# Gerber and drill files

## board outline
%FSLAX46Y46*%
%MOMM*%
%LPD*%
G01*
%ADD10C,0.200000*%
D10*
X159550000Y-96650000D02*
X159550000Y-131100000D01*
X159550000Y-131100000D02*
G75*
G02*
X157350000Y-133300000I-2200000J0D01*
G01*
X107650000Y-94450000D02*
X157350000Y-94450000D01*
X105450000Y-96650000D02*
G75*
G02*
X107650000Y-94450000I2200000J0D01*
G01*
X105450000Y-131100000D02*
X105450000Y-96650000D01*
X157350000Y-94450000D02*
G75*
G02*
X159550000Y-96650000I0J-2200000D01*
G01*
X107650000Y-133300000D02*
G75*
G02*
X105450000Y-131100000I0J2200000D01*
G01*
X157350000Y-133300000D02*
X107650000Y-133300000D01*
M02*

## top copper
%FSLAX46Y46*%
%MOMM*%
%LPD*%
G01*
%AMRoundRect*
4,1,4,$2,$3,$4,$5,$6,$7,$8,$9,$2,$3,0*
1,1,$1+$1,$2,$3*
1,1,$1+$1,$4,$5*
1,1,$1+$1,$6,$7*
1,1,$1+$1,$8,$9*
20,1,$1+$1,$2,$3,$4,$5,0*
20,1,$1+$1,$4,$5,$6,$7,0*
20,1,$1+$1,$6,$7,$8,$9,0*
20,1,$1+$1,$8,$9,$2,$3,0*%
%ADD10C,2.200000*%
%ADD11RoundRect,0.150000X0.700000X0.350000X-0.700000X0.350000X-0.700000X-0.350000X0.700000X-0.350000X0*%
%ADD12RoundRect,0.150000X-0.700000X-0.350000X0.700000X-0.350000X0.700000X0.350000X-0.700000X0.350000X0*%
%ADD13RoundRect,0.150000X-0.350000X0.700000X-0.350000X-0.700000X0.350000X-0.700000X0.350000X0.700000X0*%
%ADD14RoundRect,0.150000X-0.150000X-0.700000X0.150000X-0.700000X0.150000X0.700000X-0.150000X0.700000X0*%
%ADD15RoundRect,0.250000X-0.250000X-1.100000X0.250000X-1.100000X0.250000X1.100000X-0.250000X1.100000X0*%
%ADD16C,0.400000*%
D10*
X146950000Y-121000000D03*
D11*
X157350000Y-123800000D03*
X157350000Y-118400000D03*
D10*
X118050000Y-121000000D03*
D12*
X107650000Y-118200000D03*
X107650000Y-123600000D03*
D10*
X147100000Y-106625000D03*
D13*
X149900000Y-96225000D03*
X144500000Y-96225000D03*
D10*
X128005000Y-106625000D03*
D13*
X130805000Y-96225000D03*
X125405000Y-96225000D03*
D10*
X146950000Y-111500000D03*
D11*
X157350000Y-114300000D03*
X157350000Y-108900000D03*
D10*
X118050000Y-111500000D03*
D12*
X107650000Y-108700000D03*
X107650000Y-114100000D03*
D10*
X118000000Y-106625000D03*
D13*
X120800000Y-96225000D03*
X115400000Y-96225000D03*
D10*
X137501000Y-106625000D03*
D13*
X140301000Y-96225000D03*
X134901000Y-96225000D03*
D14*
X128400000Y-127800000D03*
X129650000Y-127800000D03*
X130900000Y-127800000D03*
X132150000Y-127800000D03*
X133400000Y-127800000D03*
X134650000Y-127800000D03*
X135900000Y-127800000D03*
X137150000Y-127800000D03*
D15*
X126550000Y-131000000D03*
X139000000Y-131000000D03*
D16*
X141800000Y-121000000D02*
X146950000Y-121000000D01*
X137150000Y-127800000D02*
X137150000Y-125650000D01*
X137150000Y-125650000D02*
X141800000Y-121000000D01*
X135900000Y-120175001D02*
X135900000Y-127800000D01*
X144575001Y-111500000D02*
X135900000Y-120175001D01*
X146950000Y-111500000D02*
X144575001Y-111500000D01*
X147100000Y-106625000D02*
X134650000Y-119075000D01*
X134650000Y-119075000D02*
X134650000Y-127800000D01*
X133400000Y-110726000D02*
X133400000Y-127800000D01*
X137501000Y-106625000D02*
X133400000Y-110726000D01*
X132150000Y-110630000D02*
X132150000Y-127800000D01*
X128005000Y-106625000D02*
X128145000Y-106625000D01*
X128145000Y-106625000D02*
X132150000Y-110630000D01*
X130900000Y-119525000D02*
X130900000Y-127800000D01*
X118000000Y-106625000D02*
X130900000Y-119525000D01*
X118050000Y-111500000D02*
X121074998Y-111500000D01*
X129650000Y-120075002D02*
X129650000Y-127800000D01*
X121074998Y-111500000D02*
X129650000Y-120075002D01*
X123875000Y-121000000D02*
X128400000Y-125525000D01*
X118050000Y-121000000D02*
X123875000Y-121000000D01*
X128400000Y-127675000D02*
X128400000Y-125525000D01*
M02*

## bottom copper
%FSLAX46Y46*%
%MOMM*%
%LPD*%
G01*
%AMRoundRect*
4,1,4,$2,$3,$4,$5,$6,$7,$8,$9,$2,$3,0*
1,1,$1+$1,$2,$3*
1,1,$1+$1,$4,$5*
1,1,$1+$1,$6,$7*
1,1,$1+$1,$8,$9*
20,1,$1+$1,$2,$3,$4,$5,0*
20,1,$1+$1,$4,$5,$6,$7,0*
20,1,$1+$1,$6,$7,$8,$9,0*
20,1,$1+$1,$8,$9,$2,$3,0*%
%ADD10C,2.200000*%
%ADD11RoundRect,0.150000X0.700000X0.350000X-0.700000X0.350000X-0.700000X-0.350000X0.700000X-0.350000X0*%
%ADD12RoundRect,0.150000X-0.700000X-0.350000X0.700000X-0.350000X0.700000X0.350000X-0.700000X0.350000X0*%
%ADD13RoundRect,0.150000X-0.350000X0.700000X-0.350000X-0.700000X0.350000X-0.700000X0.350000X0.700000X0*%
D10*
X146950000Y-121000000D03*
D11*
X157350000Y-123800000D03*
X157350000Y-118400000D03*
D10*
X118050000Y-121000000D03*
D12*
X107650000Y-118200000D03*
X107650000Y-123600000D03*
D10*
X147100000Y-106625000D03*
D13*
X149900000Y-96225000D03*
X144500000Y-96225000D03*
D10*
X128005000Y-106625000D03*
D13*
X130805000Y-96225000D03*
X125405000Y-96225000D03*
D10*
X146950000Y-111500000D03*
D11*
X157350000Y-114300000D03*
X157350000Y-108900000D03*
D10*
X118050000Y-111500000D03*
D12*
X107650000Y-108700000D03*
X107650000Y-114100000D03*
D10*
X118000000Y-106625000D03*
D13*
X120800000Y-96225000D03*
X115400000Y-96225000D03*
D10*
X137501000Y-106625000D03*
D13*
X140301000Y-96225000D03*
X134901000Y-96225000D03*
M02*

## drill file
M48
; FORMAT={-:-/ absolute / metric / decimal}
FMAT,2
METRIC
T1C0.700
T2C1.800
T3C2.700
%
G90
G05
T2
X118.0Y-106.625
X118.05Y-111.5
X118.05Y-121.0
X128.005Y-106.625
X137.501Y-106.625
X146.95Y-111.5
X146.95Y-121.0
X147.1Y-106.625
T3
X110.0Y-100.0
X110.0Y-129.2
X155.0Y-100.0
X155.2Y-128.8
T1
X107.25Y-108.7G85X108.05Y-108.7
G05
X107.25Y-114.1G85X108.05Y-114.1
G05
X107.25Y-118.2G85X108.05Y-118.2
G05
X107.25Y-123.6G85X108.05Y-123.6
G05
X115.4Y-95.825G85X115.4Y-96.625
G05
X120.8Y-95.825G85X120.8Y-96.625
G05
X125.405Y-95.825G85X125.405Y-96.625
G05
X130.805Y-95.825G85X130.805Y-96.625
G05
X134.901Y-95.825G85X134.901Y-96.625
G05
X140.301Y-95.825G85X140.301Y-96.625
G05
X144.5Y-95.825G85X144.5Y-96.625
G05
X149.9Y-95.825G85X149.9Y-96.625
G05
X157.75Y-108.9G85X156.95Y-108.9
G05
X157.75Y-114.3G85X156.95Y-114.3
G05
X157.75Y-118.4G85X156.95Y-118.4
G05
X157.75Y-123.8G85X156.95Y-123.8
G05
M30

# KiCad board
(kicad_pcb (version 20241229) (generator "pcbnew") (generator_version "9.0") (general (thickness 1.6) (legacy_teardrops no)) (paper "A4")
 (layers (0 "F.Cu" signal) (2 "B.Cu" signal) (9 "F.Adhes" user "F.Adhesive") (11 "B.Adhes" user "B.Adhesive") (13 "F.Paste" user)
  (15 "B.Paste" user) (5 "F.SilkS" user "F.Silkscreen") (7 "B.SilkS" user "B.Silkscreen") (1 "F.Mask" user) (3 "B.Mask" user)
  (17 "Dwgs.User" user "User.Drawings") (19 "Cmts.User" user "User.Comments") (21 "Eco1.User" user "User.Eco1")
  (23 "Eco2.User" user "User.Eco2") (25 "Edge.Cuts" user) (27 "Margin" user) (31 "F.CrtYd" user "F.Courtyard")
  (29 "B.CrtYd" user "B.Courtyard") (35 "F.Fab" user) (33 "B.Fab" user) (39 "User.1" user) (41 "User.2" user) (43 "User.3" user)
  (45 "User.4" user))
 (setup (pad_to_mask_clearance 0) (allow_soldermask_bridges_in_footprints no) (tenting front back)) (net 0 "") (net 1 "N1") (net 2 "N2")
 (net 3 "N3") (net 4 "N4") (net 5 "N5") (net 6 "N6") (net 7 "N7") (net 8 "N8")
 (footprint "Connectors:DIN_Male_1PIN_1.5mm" (layer "F.Cu") (at 152 120.5 180)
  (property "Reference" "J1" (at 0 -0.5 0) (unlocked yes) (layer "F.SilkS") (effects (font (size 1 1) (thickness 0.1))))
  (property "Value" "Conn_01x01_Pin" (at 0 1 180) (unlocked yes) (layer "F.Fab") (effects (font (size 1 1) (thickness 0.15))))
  (pad "1" thru_hole circle (at 5.05 -0.5 180) (size 2.2 2.2) (drill 1.8) (layers "*.Cu" "*.Mask") (remove_unused_layers no) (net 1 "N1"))
  (pad "3" thru_hole roundrect (at -5.35 -3.3 180) (size 1.7 1) (drill oval 1.5 0.7) (layers "*.Cu" "*.Mask") (remove_unused_layers no)
   (roundrect_rratio 0.15))
  (pad "3" thru_hole roundrect (at -5.35 2.1 180) (size 1.7 1) (drill oval 1.5 0.7) (layers "*.Cu" "*.Mask") (remove_unused_layers no)
   (roundrect_rratio 0.15)))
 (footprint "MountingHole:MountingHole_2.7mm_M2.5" (layer "F.Cu") (at 110 129.2)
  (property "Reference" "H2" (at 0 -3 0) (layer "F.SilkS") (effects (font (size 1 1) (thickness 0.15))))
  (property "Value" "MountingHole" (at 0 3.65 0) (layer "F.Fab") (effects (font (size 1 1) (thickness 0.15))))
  (pad "" np_thru_hole circle (at 0 0) (size 2.7 2.7) (drill 2.7) (layers "*.Cu" "*.Mask")))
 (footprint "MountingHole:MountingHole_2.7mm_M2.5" (layer "F.Cu") (at 155.2 128.8)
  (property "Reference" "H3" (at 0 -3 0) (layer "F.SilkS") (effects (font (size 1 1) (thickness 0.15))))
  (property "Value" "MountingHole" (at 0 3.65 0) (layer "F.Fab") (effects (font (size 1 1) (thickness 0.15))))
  (pad "" np_thru_hole circle (at 0 0) (size 2.7 2.7) (drill 2.7) (layers "*.Cu" "*.Mask")))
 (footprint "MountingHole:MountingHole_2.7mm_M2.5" (layer "F.Cu") (at 110 100 90)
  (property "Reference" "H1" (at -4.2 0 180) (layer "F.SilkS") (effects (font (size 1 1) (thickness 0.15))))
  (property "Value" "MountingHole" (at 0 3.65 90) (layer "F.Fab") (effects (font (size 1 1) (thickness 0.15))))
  (pad "" np_thru_hole circle (at 0 0 90) (size 2.7 2.7) (drill 2.7) (layers "*.Cu" "*.Mask")))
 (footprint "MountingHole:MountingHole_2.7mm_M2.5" (layer "F.Cu") (at 155 100 90)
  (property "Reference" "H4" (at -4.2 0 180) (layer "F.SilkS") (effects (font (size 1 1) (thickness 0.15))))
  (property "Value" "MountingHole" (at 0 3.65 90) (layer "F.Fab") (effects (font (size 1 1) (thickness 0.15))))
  (pad "" np_thru_hole circle (at 0 0 90) (size 2.7 2.7) (drill 2.7) (layers "*.Cu" "*.Mask")))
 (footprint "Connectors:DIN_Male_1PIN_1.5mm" (layer "F.Cu") (at 113 121.5)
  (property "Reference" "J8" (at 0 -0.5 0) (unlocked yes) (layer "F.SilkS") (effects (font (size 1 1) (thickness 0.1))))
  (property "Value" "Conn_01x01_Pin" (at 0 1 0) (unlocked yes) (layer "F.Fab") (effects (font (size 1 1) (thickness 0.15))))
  (pad "1" thru_hole circle (at 5.05 -0.5) (size 2.2 2.2) (drill 1.8) (layers "*.Cu" "*.Mask") (remove_unused_layers no) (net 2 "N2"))
  (pad "3" thru_hole roundrect (at -5.35 -3.3) (size 1.7 1) (drill oval 1.5 0.7) (layers "*.Cu" "*.Mask") (remove_unused_layers no)
   (roundrect_rratio 0.15))
  (pad "3" thru_hole roundrect (at -5.35 2.1) (size 1.7 1) (drill oval 1.5 0.7) (layers "*.Cu" "*.Mask") (remove_unused_layers no)
   (roundrect_rratio 0.15)))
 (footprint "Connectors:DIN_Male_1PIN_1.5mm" (layer "F.Cu") (at 146.6 101.575 -90)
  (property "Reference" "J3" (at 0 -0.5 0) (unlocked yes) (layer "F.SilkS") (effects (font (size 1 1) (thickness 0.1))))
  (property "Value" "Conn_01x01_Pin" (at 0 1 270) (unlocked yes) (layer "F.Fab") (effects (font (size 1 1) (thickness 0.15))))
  (pad "1" thru_hole circle (at 5.05 -0.5 270) (size 2.2 2.2) (drill 1.8) (layers "*.Cu" "*.Mask") (remove_unused_layers no) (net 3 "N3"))
  (pad "3" thru_hole roundrect (at -5.35 -3.3 270) (size 1.7 1) (drill oval 1.5 0.7) (layers "*.Cu" "*.Mask") (remove_unused_layers no)
   (roundrect_rratio 0.15))
  (pad "3" thru_hole roundrect (at -5.35 2.1 270) (size 1.7 1) (drill oval 1.5 0.7) (layers "*.Cu" "*.Mask") (remove_unused_layers no)
   (roundrect_rratio 0.15)))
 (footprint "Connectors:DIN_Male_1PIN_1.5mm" (layer "F.Cu") (at 127.505 101.575 -90)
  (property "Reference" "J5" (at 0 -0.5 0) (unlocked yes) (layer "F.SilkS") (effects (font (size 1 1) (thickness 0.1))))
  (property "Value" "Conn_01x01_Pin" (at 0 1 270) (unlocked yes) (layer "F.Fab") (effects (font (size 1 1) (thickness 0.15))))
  (pad "1" thru_hole circle (at 5.05 -0.5 270) (size 2.2 2.2) (drill 1.8) (layers "*.Cu" "*.Mask") (remove_unused_layers no) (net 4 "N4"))
  (pad "3" thru_hole roundrect (at -5.35 -3.3 270) (size 1.7 1) (drill oval 1.5 0.7) (layers "*.Cu" "*.Mask") (remove_unused_layers no)
   (roundrect_rratio 0.15))
  (pad "3" thru_hole roundrect (at -5.35 2.1 270) (size 1.7 1) (drill oval 1.5 0.7) (layers "*.Cu" "*.Mask") (remove_unused_layers no)
   (roundrect_rratio 0.15)))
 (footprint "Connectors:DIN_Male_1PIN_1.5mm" (layer "F.Cu") (at 152 111 180)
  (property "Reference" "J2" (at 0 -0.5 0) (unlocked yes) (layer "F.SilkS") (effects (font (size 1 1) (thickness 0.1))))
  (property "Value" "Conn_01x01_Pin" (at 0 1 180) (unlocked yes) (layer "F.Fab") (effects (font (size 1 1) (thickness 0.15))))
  (pad "1" thru_hole circle (at 5.05 -0.5 180) (size 2.2 2.2) (drill 1.8) (layers "*.Cu" "*.Mask") (remove_unused_layers no) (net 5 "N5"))
  (pad "3" thru_hole roundrect (at -5.35 -3.3 180) (size 1.7 1) (drill oval 1.5 0.7) (layers "*.Cu" "*.Mask") (remove_unused_layers no)
   (roundrect_rratio 0.15))
  (pad "3" thru_hole roundrect (at -5.35 2.1 180) (size 1.7 1) (drill oval 1.5 0.7) (layers "*.Cu" "*.Mask") (remove_unused_layers no)
   (roundrect_rratio 0.15)))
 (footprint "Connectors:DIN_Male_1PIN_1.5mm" (layer "F.Cu") (at 113 112)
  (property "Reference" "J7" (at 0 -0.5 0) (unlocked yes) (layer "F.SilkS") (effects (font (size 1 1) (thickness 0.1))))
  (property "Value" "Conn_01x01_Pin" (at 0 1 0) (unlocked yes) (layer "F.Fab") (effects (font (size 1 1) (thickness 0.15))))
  (pad "1" thru_hole circle (at 5.05 -0.5) (size 2.2 2.2) (drill 1.8) (layers "*.Cu" "*.Mask") (remove_unused_layers no) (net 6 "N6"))
  (pad "3" thru_hole roundrect (at -5.35 -3.3) (size 1.7 1) (drill oval 1.5 0.7) (layers "*.Cu" "*.Mask") (remove_unused_layers no)
   (roundrect_rratio 0.15))
  (pad "3" thru_hole roundrect (at -5.35 2.1) (size 1.7 1) (drill oval 1.5 0.7) (layers "*.Cu" "*.Mask") (remove_unused_layers no)
   (roundrect_rratio 0.15)))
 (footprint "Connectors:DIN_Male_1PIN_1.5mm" (layer "F.Cu") (at 117.5 101.575 -90)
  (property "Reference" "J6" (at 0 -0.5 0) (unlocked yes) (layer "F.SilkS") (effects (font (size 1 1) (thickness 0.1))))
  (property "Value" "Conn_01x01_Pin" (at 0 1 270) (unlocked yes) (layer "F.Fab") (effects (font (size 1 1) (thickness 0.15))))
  (pad "1" thru_hole circle (at 5.05 -0.5 270) (size 2.2 2.2) (drill 1.8) (layers "*.Cu" "*.Mask") (remove_unused_layers no) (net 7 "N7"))
  (pad "3" thru_hole roundrect (at -5.35 -3.3 270) (size 1.7 1) (drill oval 1.5 0.7) (layers "*.Cu" "*.Mask") (remove_unused_layers no)
   (roundrect_rratio 0.15))
  (pad "3" thru_hole roundrect (at -5.35 2.1 270) (size 1.7 1) (drill oval 1.5 0.7) (layers "*.Cu" "*.Mask") (remove_unused_layers no)
   (roundrect_rratio 0.15)))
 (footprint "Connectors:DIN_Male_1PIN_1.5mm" (layer "F.Cu") (at 137.001 101.575 -90)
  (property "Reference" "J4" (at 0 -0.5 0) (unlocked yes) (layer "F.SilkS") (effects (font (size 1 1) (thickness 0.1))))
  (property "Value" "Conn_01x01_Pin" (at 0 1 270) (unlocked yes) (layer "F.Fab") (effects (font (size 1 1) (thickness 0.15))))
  (pad "1" thru_hole circle (at 5.05 -0.5 270) (size 2.2 2.2) (drill 1.8) (layers "*.Cu" "*.Mask") (remove_unused_layers no) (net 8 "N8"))
  (pad "3" thru_hole roundrect (at -5.35 -3.3 270) (size 1.7 1) (drill oval 1.5 0.7) (layers "*.Cu" "*.Mask") (remove_unused_layers no)
   (roundrect_rratio 0.15))
  (pad "3" thru_hole roundrect (at -5.35 2.1 270) (size 1.7 1) (drill oval 1.5 0.7) (layers "*.Cu" "*.Mask") (remove_unused_layers no)
   (roundrect_rratio 0.15)))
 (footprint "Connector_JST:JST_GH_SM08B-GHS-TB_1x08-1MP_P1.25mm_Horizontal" (layer "F.Cu") (at 132.775 129.65)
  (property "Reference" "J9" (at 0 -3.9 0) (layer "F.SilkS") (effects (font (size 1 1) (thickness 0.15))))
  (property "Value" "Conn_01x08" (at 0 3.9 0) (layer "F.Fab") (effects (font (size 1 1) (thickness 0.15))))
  (pad "1" smd roundrect (at -4.375 -1.85) (size 0.6 1.7) (layers "F.Cu" "F.Mask" "F.Paste") (roundrect_rratio 0.25) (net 2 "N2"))
  (pad "2" smd roundrect (at -3.125 -1.85) (size 0.6 1.7) (layers "F.Cu" "F.Mask" "F.Paste") (roundrect_rratio 0.25) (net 6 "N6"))
  (pad "3" smd roundrect (at -1.875 -1.85) (size 0.6 1.7) (layers "F.Cu" "F.Mask" "F.Paste") (roundrect_rratio 0.25) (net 7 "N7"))
  (pad "4" smd roundrect (at -0.625 -1.85) (size 0.6 1.7) (layers "F.Cu" "F.Mask" "F.Paste") (roundrect_rratio 0.25) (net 4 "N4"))
  (pad "5" smd roundrect (at 0.625 -1.85) (size 0.6 1.7) (layers "F.Cu" "F.Mask" "F.Paste") (roundrect_rratio 0.25) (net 8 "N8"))
  (pad "6" smd roundrect (at 1.875 -1.85) (size 0.6 1.7) (layers "F.Cu" "F.Mask" "F.Paste") (roundrect_rratio 0.25) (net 3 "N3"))
  (pad "7" smd roundrect (at 3.125 -1.85) (size 0.6 1.7) (layers "F.Cu" "F.Mask" "F.Paste") (roundrect_rratio 0.25) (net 5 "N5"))
  (pad "8" smd roundrect (at 4.375 -1.85) (size 0.6 1.7) (layers "F.Cu" "F.Mask" "F.Paste") (roundrect_rratio 0.25) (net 1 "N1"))
  (pad "MP" smd roundrect (at -6.225 1.35) (size 1 2.7) (layers "F.Cu" "F.Mask" "F.Paste") (roundrect_rratio 0.25))
  (pad "MP" smd roundrect (at 6.225 1.35) (size 1 2.7) (layers "F.Cu" "F.Mask" "F.Paste") (roundrect_rratio 0.25)))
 (gr_line (start 159.55 96.65) (end 159.55 131.1) (stroke (width 0.2) (type default)) (layer "Edge.Cuts"))
 (gr_arc (start 159.55 131.1) (mid 158.905635 132.655635) (end 157.35 133.3) (stroke (width 0.2) (type default)) (layer "Edge.Cuts"))
 (gr_line (start 107.65 94.45) (end 157.35 94.45) (stroke (width 0.2) (type default)) (layer "Edge.Cuts"))
 (gr_arc (start 105.45 96.65) (mid 106.094365 95.094365) (end 107.65 94.45) (stroke (width 0.2) (type default)) (layer "Edge.Cuts"))
 (gr_line (start 105.45 131.1) (end 105.45 96.65) (stroke (width 0.2) (type default)) (layer "Edge.Cuts"))
 (gr_arc (start 157.35 94.45) (mid 158.905635 95.094365) (end 159.55 96.65) (stroke (width 0.2) (type default)) (layer "Edge.Cuts"))
 (gr_arc (start 107.65 133.3) (mid 106.094365 132.655635) (end 105.45 131.1) (stroke (width 0.2) (type default)) (layer "Edge.Cuts"))
 (gr_line (start 157.35 133.3) (end 107.65 133.3) (stroke (width 0.2) (type default)) (layer "Edge.Cuts"))
 (segment (start 141.8 121) (end 146.95 121) (width 0.4) (layer "F.Cu") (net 1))
 (segment (start 137.15 127.8) (end 137.15 125.65) (width 0.4) (layer "F.Cu") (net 1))
 (segment (start 137.15 125.65) (end 141.8 121) (width 0.4) (layer "F.Cu") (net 1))
 (segment (start 135.9 120.175001) (end 135.9 127.8) (width 0.4) (layer "F.Cu") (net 5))
 (segment (start 144.575001 111.5) (end 135.9 120.175001) (width 0.4) (layer "F.Cu") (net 5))
 (segment (start 146.95 111.5) (end 144.575001 111.5) (width 0.4) (layer "F.Cu") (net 5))
 (segment (start 147.1 106.625) (end 134.65 119.075) (width 0.4) (layer "F.Cu") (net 3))
 (segment (start 134.65 119.075) (end 134.65 127.8) (width 0.4) (layer "F.Cu") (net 3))
 (segment (start 133.4 110.726) (end 133.4 127.8) (width 0.4) (layer "F.Cu") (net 8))
 (segment (start 137.501 106.625) (end 133.4 110.726) (width 0.4) (layer "F.Cu") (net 8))
 (segment (start 132.15 110.63) (end 132.15 127.8) (width 0.4) (layer "F.Cu") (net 4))
 (segment (start 128.005 106.625) (end 128.145 106.625) (width 0.4) (layer "F.Cu") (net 4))
 (segment (start 128.145 106.625) (end 132.15 110.63) (width 0.4) (layer "F.Cu") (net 4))
 (segment (start 130.9 119.525) (end 130.9 127.8) (width 0.4) (layer "F.Cu") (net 7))
 (segment (start 118 106.625) (end 130.9 119.525) (width 0.4) (layer "F.Cu") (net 7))
 (segment (start 118.05 111.5) (end 121.074998 111.5) (width 0.4) (layer "F.Cu") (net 6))
 (segment (start 129.65 120.075002) (end 129.65 127.8) (width 0.4) (layer "F.Cu") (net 6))
 (segment (start 121.074998 111.5) (end 129.65 120.075002) (width 0.4) (layer "F.Cu") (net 6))
 (segment (start 123.875 121) (end 128.4 125.525) (width 0.4) (layer "F.Cu") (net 2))
 (segment (start 118.05 121) (end 123.875 121) (width 0.4) (layer "F.Cu") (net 2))
 (segment (start 128.4 127.675) (end 128.4 125.525) (width 0.4) (layer "F.Cu") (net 2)))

